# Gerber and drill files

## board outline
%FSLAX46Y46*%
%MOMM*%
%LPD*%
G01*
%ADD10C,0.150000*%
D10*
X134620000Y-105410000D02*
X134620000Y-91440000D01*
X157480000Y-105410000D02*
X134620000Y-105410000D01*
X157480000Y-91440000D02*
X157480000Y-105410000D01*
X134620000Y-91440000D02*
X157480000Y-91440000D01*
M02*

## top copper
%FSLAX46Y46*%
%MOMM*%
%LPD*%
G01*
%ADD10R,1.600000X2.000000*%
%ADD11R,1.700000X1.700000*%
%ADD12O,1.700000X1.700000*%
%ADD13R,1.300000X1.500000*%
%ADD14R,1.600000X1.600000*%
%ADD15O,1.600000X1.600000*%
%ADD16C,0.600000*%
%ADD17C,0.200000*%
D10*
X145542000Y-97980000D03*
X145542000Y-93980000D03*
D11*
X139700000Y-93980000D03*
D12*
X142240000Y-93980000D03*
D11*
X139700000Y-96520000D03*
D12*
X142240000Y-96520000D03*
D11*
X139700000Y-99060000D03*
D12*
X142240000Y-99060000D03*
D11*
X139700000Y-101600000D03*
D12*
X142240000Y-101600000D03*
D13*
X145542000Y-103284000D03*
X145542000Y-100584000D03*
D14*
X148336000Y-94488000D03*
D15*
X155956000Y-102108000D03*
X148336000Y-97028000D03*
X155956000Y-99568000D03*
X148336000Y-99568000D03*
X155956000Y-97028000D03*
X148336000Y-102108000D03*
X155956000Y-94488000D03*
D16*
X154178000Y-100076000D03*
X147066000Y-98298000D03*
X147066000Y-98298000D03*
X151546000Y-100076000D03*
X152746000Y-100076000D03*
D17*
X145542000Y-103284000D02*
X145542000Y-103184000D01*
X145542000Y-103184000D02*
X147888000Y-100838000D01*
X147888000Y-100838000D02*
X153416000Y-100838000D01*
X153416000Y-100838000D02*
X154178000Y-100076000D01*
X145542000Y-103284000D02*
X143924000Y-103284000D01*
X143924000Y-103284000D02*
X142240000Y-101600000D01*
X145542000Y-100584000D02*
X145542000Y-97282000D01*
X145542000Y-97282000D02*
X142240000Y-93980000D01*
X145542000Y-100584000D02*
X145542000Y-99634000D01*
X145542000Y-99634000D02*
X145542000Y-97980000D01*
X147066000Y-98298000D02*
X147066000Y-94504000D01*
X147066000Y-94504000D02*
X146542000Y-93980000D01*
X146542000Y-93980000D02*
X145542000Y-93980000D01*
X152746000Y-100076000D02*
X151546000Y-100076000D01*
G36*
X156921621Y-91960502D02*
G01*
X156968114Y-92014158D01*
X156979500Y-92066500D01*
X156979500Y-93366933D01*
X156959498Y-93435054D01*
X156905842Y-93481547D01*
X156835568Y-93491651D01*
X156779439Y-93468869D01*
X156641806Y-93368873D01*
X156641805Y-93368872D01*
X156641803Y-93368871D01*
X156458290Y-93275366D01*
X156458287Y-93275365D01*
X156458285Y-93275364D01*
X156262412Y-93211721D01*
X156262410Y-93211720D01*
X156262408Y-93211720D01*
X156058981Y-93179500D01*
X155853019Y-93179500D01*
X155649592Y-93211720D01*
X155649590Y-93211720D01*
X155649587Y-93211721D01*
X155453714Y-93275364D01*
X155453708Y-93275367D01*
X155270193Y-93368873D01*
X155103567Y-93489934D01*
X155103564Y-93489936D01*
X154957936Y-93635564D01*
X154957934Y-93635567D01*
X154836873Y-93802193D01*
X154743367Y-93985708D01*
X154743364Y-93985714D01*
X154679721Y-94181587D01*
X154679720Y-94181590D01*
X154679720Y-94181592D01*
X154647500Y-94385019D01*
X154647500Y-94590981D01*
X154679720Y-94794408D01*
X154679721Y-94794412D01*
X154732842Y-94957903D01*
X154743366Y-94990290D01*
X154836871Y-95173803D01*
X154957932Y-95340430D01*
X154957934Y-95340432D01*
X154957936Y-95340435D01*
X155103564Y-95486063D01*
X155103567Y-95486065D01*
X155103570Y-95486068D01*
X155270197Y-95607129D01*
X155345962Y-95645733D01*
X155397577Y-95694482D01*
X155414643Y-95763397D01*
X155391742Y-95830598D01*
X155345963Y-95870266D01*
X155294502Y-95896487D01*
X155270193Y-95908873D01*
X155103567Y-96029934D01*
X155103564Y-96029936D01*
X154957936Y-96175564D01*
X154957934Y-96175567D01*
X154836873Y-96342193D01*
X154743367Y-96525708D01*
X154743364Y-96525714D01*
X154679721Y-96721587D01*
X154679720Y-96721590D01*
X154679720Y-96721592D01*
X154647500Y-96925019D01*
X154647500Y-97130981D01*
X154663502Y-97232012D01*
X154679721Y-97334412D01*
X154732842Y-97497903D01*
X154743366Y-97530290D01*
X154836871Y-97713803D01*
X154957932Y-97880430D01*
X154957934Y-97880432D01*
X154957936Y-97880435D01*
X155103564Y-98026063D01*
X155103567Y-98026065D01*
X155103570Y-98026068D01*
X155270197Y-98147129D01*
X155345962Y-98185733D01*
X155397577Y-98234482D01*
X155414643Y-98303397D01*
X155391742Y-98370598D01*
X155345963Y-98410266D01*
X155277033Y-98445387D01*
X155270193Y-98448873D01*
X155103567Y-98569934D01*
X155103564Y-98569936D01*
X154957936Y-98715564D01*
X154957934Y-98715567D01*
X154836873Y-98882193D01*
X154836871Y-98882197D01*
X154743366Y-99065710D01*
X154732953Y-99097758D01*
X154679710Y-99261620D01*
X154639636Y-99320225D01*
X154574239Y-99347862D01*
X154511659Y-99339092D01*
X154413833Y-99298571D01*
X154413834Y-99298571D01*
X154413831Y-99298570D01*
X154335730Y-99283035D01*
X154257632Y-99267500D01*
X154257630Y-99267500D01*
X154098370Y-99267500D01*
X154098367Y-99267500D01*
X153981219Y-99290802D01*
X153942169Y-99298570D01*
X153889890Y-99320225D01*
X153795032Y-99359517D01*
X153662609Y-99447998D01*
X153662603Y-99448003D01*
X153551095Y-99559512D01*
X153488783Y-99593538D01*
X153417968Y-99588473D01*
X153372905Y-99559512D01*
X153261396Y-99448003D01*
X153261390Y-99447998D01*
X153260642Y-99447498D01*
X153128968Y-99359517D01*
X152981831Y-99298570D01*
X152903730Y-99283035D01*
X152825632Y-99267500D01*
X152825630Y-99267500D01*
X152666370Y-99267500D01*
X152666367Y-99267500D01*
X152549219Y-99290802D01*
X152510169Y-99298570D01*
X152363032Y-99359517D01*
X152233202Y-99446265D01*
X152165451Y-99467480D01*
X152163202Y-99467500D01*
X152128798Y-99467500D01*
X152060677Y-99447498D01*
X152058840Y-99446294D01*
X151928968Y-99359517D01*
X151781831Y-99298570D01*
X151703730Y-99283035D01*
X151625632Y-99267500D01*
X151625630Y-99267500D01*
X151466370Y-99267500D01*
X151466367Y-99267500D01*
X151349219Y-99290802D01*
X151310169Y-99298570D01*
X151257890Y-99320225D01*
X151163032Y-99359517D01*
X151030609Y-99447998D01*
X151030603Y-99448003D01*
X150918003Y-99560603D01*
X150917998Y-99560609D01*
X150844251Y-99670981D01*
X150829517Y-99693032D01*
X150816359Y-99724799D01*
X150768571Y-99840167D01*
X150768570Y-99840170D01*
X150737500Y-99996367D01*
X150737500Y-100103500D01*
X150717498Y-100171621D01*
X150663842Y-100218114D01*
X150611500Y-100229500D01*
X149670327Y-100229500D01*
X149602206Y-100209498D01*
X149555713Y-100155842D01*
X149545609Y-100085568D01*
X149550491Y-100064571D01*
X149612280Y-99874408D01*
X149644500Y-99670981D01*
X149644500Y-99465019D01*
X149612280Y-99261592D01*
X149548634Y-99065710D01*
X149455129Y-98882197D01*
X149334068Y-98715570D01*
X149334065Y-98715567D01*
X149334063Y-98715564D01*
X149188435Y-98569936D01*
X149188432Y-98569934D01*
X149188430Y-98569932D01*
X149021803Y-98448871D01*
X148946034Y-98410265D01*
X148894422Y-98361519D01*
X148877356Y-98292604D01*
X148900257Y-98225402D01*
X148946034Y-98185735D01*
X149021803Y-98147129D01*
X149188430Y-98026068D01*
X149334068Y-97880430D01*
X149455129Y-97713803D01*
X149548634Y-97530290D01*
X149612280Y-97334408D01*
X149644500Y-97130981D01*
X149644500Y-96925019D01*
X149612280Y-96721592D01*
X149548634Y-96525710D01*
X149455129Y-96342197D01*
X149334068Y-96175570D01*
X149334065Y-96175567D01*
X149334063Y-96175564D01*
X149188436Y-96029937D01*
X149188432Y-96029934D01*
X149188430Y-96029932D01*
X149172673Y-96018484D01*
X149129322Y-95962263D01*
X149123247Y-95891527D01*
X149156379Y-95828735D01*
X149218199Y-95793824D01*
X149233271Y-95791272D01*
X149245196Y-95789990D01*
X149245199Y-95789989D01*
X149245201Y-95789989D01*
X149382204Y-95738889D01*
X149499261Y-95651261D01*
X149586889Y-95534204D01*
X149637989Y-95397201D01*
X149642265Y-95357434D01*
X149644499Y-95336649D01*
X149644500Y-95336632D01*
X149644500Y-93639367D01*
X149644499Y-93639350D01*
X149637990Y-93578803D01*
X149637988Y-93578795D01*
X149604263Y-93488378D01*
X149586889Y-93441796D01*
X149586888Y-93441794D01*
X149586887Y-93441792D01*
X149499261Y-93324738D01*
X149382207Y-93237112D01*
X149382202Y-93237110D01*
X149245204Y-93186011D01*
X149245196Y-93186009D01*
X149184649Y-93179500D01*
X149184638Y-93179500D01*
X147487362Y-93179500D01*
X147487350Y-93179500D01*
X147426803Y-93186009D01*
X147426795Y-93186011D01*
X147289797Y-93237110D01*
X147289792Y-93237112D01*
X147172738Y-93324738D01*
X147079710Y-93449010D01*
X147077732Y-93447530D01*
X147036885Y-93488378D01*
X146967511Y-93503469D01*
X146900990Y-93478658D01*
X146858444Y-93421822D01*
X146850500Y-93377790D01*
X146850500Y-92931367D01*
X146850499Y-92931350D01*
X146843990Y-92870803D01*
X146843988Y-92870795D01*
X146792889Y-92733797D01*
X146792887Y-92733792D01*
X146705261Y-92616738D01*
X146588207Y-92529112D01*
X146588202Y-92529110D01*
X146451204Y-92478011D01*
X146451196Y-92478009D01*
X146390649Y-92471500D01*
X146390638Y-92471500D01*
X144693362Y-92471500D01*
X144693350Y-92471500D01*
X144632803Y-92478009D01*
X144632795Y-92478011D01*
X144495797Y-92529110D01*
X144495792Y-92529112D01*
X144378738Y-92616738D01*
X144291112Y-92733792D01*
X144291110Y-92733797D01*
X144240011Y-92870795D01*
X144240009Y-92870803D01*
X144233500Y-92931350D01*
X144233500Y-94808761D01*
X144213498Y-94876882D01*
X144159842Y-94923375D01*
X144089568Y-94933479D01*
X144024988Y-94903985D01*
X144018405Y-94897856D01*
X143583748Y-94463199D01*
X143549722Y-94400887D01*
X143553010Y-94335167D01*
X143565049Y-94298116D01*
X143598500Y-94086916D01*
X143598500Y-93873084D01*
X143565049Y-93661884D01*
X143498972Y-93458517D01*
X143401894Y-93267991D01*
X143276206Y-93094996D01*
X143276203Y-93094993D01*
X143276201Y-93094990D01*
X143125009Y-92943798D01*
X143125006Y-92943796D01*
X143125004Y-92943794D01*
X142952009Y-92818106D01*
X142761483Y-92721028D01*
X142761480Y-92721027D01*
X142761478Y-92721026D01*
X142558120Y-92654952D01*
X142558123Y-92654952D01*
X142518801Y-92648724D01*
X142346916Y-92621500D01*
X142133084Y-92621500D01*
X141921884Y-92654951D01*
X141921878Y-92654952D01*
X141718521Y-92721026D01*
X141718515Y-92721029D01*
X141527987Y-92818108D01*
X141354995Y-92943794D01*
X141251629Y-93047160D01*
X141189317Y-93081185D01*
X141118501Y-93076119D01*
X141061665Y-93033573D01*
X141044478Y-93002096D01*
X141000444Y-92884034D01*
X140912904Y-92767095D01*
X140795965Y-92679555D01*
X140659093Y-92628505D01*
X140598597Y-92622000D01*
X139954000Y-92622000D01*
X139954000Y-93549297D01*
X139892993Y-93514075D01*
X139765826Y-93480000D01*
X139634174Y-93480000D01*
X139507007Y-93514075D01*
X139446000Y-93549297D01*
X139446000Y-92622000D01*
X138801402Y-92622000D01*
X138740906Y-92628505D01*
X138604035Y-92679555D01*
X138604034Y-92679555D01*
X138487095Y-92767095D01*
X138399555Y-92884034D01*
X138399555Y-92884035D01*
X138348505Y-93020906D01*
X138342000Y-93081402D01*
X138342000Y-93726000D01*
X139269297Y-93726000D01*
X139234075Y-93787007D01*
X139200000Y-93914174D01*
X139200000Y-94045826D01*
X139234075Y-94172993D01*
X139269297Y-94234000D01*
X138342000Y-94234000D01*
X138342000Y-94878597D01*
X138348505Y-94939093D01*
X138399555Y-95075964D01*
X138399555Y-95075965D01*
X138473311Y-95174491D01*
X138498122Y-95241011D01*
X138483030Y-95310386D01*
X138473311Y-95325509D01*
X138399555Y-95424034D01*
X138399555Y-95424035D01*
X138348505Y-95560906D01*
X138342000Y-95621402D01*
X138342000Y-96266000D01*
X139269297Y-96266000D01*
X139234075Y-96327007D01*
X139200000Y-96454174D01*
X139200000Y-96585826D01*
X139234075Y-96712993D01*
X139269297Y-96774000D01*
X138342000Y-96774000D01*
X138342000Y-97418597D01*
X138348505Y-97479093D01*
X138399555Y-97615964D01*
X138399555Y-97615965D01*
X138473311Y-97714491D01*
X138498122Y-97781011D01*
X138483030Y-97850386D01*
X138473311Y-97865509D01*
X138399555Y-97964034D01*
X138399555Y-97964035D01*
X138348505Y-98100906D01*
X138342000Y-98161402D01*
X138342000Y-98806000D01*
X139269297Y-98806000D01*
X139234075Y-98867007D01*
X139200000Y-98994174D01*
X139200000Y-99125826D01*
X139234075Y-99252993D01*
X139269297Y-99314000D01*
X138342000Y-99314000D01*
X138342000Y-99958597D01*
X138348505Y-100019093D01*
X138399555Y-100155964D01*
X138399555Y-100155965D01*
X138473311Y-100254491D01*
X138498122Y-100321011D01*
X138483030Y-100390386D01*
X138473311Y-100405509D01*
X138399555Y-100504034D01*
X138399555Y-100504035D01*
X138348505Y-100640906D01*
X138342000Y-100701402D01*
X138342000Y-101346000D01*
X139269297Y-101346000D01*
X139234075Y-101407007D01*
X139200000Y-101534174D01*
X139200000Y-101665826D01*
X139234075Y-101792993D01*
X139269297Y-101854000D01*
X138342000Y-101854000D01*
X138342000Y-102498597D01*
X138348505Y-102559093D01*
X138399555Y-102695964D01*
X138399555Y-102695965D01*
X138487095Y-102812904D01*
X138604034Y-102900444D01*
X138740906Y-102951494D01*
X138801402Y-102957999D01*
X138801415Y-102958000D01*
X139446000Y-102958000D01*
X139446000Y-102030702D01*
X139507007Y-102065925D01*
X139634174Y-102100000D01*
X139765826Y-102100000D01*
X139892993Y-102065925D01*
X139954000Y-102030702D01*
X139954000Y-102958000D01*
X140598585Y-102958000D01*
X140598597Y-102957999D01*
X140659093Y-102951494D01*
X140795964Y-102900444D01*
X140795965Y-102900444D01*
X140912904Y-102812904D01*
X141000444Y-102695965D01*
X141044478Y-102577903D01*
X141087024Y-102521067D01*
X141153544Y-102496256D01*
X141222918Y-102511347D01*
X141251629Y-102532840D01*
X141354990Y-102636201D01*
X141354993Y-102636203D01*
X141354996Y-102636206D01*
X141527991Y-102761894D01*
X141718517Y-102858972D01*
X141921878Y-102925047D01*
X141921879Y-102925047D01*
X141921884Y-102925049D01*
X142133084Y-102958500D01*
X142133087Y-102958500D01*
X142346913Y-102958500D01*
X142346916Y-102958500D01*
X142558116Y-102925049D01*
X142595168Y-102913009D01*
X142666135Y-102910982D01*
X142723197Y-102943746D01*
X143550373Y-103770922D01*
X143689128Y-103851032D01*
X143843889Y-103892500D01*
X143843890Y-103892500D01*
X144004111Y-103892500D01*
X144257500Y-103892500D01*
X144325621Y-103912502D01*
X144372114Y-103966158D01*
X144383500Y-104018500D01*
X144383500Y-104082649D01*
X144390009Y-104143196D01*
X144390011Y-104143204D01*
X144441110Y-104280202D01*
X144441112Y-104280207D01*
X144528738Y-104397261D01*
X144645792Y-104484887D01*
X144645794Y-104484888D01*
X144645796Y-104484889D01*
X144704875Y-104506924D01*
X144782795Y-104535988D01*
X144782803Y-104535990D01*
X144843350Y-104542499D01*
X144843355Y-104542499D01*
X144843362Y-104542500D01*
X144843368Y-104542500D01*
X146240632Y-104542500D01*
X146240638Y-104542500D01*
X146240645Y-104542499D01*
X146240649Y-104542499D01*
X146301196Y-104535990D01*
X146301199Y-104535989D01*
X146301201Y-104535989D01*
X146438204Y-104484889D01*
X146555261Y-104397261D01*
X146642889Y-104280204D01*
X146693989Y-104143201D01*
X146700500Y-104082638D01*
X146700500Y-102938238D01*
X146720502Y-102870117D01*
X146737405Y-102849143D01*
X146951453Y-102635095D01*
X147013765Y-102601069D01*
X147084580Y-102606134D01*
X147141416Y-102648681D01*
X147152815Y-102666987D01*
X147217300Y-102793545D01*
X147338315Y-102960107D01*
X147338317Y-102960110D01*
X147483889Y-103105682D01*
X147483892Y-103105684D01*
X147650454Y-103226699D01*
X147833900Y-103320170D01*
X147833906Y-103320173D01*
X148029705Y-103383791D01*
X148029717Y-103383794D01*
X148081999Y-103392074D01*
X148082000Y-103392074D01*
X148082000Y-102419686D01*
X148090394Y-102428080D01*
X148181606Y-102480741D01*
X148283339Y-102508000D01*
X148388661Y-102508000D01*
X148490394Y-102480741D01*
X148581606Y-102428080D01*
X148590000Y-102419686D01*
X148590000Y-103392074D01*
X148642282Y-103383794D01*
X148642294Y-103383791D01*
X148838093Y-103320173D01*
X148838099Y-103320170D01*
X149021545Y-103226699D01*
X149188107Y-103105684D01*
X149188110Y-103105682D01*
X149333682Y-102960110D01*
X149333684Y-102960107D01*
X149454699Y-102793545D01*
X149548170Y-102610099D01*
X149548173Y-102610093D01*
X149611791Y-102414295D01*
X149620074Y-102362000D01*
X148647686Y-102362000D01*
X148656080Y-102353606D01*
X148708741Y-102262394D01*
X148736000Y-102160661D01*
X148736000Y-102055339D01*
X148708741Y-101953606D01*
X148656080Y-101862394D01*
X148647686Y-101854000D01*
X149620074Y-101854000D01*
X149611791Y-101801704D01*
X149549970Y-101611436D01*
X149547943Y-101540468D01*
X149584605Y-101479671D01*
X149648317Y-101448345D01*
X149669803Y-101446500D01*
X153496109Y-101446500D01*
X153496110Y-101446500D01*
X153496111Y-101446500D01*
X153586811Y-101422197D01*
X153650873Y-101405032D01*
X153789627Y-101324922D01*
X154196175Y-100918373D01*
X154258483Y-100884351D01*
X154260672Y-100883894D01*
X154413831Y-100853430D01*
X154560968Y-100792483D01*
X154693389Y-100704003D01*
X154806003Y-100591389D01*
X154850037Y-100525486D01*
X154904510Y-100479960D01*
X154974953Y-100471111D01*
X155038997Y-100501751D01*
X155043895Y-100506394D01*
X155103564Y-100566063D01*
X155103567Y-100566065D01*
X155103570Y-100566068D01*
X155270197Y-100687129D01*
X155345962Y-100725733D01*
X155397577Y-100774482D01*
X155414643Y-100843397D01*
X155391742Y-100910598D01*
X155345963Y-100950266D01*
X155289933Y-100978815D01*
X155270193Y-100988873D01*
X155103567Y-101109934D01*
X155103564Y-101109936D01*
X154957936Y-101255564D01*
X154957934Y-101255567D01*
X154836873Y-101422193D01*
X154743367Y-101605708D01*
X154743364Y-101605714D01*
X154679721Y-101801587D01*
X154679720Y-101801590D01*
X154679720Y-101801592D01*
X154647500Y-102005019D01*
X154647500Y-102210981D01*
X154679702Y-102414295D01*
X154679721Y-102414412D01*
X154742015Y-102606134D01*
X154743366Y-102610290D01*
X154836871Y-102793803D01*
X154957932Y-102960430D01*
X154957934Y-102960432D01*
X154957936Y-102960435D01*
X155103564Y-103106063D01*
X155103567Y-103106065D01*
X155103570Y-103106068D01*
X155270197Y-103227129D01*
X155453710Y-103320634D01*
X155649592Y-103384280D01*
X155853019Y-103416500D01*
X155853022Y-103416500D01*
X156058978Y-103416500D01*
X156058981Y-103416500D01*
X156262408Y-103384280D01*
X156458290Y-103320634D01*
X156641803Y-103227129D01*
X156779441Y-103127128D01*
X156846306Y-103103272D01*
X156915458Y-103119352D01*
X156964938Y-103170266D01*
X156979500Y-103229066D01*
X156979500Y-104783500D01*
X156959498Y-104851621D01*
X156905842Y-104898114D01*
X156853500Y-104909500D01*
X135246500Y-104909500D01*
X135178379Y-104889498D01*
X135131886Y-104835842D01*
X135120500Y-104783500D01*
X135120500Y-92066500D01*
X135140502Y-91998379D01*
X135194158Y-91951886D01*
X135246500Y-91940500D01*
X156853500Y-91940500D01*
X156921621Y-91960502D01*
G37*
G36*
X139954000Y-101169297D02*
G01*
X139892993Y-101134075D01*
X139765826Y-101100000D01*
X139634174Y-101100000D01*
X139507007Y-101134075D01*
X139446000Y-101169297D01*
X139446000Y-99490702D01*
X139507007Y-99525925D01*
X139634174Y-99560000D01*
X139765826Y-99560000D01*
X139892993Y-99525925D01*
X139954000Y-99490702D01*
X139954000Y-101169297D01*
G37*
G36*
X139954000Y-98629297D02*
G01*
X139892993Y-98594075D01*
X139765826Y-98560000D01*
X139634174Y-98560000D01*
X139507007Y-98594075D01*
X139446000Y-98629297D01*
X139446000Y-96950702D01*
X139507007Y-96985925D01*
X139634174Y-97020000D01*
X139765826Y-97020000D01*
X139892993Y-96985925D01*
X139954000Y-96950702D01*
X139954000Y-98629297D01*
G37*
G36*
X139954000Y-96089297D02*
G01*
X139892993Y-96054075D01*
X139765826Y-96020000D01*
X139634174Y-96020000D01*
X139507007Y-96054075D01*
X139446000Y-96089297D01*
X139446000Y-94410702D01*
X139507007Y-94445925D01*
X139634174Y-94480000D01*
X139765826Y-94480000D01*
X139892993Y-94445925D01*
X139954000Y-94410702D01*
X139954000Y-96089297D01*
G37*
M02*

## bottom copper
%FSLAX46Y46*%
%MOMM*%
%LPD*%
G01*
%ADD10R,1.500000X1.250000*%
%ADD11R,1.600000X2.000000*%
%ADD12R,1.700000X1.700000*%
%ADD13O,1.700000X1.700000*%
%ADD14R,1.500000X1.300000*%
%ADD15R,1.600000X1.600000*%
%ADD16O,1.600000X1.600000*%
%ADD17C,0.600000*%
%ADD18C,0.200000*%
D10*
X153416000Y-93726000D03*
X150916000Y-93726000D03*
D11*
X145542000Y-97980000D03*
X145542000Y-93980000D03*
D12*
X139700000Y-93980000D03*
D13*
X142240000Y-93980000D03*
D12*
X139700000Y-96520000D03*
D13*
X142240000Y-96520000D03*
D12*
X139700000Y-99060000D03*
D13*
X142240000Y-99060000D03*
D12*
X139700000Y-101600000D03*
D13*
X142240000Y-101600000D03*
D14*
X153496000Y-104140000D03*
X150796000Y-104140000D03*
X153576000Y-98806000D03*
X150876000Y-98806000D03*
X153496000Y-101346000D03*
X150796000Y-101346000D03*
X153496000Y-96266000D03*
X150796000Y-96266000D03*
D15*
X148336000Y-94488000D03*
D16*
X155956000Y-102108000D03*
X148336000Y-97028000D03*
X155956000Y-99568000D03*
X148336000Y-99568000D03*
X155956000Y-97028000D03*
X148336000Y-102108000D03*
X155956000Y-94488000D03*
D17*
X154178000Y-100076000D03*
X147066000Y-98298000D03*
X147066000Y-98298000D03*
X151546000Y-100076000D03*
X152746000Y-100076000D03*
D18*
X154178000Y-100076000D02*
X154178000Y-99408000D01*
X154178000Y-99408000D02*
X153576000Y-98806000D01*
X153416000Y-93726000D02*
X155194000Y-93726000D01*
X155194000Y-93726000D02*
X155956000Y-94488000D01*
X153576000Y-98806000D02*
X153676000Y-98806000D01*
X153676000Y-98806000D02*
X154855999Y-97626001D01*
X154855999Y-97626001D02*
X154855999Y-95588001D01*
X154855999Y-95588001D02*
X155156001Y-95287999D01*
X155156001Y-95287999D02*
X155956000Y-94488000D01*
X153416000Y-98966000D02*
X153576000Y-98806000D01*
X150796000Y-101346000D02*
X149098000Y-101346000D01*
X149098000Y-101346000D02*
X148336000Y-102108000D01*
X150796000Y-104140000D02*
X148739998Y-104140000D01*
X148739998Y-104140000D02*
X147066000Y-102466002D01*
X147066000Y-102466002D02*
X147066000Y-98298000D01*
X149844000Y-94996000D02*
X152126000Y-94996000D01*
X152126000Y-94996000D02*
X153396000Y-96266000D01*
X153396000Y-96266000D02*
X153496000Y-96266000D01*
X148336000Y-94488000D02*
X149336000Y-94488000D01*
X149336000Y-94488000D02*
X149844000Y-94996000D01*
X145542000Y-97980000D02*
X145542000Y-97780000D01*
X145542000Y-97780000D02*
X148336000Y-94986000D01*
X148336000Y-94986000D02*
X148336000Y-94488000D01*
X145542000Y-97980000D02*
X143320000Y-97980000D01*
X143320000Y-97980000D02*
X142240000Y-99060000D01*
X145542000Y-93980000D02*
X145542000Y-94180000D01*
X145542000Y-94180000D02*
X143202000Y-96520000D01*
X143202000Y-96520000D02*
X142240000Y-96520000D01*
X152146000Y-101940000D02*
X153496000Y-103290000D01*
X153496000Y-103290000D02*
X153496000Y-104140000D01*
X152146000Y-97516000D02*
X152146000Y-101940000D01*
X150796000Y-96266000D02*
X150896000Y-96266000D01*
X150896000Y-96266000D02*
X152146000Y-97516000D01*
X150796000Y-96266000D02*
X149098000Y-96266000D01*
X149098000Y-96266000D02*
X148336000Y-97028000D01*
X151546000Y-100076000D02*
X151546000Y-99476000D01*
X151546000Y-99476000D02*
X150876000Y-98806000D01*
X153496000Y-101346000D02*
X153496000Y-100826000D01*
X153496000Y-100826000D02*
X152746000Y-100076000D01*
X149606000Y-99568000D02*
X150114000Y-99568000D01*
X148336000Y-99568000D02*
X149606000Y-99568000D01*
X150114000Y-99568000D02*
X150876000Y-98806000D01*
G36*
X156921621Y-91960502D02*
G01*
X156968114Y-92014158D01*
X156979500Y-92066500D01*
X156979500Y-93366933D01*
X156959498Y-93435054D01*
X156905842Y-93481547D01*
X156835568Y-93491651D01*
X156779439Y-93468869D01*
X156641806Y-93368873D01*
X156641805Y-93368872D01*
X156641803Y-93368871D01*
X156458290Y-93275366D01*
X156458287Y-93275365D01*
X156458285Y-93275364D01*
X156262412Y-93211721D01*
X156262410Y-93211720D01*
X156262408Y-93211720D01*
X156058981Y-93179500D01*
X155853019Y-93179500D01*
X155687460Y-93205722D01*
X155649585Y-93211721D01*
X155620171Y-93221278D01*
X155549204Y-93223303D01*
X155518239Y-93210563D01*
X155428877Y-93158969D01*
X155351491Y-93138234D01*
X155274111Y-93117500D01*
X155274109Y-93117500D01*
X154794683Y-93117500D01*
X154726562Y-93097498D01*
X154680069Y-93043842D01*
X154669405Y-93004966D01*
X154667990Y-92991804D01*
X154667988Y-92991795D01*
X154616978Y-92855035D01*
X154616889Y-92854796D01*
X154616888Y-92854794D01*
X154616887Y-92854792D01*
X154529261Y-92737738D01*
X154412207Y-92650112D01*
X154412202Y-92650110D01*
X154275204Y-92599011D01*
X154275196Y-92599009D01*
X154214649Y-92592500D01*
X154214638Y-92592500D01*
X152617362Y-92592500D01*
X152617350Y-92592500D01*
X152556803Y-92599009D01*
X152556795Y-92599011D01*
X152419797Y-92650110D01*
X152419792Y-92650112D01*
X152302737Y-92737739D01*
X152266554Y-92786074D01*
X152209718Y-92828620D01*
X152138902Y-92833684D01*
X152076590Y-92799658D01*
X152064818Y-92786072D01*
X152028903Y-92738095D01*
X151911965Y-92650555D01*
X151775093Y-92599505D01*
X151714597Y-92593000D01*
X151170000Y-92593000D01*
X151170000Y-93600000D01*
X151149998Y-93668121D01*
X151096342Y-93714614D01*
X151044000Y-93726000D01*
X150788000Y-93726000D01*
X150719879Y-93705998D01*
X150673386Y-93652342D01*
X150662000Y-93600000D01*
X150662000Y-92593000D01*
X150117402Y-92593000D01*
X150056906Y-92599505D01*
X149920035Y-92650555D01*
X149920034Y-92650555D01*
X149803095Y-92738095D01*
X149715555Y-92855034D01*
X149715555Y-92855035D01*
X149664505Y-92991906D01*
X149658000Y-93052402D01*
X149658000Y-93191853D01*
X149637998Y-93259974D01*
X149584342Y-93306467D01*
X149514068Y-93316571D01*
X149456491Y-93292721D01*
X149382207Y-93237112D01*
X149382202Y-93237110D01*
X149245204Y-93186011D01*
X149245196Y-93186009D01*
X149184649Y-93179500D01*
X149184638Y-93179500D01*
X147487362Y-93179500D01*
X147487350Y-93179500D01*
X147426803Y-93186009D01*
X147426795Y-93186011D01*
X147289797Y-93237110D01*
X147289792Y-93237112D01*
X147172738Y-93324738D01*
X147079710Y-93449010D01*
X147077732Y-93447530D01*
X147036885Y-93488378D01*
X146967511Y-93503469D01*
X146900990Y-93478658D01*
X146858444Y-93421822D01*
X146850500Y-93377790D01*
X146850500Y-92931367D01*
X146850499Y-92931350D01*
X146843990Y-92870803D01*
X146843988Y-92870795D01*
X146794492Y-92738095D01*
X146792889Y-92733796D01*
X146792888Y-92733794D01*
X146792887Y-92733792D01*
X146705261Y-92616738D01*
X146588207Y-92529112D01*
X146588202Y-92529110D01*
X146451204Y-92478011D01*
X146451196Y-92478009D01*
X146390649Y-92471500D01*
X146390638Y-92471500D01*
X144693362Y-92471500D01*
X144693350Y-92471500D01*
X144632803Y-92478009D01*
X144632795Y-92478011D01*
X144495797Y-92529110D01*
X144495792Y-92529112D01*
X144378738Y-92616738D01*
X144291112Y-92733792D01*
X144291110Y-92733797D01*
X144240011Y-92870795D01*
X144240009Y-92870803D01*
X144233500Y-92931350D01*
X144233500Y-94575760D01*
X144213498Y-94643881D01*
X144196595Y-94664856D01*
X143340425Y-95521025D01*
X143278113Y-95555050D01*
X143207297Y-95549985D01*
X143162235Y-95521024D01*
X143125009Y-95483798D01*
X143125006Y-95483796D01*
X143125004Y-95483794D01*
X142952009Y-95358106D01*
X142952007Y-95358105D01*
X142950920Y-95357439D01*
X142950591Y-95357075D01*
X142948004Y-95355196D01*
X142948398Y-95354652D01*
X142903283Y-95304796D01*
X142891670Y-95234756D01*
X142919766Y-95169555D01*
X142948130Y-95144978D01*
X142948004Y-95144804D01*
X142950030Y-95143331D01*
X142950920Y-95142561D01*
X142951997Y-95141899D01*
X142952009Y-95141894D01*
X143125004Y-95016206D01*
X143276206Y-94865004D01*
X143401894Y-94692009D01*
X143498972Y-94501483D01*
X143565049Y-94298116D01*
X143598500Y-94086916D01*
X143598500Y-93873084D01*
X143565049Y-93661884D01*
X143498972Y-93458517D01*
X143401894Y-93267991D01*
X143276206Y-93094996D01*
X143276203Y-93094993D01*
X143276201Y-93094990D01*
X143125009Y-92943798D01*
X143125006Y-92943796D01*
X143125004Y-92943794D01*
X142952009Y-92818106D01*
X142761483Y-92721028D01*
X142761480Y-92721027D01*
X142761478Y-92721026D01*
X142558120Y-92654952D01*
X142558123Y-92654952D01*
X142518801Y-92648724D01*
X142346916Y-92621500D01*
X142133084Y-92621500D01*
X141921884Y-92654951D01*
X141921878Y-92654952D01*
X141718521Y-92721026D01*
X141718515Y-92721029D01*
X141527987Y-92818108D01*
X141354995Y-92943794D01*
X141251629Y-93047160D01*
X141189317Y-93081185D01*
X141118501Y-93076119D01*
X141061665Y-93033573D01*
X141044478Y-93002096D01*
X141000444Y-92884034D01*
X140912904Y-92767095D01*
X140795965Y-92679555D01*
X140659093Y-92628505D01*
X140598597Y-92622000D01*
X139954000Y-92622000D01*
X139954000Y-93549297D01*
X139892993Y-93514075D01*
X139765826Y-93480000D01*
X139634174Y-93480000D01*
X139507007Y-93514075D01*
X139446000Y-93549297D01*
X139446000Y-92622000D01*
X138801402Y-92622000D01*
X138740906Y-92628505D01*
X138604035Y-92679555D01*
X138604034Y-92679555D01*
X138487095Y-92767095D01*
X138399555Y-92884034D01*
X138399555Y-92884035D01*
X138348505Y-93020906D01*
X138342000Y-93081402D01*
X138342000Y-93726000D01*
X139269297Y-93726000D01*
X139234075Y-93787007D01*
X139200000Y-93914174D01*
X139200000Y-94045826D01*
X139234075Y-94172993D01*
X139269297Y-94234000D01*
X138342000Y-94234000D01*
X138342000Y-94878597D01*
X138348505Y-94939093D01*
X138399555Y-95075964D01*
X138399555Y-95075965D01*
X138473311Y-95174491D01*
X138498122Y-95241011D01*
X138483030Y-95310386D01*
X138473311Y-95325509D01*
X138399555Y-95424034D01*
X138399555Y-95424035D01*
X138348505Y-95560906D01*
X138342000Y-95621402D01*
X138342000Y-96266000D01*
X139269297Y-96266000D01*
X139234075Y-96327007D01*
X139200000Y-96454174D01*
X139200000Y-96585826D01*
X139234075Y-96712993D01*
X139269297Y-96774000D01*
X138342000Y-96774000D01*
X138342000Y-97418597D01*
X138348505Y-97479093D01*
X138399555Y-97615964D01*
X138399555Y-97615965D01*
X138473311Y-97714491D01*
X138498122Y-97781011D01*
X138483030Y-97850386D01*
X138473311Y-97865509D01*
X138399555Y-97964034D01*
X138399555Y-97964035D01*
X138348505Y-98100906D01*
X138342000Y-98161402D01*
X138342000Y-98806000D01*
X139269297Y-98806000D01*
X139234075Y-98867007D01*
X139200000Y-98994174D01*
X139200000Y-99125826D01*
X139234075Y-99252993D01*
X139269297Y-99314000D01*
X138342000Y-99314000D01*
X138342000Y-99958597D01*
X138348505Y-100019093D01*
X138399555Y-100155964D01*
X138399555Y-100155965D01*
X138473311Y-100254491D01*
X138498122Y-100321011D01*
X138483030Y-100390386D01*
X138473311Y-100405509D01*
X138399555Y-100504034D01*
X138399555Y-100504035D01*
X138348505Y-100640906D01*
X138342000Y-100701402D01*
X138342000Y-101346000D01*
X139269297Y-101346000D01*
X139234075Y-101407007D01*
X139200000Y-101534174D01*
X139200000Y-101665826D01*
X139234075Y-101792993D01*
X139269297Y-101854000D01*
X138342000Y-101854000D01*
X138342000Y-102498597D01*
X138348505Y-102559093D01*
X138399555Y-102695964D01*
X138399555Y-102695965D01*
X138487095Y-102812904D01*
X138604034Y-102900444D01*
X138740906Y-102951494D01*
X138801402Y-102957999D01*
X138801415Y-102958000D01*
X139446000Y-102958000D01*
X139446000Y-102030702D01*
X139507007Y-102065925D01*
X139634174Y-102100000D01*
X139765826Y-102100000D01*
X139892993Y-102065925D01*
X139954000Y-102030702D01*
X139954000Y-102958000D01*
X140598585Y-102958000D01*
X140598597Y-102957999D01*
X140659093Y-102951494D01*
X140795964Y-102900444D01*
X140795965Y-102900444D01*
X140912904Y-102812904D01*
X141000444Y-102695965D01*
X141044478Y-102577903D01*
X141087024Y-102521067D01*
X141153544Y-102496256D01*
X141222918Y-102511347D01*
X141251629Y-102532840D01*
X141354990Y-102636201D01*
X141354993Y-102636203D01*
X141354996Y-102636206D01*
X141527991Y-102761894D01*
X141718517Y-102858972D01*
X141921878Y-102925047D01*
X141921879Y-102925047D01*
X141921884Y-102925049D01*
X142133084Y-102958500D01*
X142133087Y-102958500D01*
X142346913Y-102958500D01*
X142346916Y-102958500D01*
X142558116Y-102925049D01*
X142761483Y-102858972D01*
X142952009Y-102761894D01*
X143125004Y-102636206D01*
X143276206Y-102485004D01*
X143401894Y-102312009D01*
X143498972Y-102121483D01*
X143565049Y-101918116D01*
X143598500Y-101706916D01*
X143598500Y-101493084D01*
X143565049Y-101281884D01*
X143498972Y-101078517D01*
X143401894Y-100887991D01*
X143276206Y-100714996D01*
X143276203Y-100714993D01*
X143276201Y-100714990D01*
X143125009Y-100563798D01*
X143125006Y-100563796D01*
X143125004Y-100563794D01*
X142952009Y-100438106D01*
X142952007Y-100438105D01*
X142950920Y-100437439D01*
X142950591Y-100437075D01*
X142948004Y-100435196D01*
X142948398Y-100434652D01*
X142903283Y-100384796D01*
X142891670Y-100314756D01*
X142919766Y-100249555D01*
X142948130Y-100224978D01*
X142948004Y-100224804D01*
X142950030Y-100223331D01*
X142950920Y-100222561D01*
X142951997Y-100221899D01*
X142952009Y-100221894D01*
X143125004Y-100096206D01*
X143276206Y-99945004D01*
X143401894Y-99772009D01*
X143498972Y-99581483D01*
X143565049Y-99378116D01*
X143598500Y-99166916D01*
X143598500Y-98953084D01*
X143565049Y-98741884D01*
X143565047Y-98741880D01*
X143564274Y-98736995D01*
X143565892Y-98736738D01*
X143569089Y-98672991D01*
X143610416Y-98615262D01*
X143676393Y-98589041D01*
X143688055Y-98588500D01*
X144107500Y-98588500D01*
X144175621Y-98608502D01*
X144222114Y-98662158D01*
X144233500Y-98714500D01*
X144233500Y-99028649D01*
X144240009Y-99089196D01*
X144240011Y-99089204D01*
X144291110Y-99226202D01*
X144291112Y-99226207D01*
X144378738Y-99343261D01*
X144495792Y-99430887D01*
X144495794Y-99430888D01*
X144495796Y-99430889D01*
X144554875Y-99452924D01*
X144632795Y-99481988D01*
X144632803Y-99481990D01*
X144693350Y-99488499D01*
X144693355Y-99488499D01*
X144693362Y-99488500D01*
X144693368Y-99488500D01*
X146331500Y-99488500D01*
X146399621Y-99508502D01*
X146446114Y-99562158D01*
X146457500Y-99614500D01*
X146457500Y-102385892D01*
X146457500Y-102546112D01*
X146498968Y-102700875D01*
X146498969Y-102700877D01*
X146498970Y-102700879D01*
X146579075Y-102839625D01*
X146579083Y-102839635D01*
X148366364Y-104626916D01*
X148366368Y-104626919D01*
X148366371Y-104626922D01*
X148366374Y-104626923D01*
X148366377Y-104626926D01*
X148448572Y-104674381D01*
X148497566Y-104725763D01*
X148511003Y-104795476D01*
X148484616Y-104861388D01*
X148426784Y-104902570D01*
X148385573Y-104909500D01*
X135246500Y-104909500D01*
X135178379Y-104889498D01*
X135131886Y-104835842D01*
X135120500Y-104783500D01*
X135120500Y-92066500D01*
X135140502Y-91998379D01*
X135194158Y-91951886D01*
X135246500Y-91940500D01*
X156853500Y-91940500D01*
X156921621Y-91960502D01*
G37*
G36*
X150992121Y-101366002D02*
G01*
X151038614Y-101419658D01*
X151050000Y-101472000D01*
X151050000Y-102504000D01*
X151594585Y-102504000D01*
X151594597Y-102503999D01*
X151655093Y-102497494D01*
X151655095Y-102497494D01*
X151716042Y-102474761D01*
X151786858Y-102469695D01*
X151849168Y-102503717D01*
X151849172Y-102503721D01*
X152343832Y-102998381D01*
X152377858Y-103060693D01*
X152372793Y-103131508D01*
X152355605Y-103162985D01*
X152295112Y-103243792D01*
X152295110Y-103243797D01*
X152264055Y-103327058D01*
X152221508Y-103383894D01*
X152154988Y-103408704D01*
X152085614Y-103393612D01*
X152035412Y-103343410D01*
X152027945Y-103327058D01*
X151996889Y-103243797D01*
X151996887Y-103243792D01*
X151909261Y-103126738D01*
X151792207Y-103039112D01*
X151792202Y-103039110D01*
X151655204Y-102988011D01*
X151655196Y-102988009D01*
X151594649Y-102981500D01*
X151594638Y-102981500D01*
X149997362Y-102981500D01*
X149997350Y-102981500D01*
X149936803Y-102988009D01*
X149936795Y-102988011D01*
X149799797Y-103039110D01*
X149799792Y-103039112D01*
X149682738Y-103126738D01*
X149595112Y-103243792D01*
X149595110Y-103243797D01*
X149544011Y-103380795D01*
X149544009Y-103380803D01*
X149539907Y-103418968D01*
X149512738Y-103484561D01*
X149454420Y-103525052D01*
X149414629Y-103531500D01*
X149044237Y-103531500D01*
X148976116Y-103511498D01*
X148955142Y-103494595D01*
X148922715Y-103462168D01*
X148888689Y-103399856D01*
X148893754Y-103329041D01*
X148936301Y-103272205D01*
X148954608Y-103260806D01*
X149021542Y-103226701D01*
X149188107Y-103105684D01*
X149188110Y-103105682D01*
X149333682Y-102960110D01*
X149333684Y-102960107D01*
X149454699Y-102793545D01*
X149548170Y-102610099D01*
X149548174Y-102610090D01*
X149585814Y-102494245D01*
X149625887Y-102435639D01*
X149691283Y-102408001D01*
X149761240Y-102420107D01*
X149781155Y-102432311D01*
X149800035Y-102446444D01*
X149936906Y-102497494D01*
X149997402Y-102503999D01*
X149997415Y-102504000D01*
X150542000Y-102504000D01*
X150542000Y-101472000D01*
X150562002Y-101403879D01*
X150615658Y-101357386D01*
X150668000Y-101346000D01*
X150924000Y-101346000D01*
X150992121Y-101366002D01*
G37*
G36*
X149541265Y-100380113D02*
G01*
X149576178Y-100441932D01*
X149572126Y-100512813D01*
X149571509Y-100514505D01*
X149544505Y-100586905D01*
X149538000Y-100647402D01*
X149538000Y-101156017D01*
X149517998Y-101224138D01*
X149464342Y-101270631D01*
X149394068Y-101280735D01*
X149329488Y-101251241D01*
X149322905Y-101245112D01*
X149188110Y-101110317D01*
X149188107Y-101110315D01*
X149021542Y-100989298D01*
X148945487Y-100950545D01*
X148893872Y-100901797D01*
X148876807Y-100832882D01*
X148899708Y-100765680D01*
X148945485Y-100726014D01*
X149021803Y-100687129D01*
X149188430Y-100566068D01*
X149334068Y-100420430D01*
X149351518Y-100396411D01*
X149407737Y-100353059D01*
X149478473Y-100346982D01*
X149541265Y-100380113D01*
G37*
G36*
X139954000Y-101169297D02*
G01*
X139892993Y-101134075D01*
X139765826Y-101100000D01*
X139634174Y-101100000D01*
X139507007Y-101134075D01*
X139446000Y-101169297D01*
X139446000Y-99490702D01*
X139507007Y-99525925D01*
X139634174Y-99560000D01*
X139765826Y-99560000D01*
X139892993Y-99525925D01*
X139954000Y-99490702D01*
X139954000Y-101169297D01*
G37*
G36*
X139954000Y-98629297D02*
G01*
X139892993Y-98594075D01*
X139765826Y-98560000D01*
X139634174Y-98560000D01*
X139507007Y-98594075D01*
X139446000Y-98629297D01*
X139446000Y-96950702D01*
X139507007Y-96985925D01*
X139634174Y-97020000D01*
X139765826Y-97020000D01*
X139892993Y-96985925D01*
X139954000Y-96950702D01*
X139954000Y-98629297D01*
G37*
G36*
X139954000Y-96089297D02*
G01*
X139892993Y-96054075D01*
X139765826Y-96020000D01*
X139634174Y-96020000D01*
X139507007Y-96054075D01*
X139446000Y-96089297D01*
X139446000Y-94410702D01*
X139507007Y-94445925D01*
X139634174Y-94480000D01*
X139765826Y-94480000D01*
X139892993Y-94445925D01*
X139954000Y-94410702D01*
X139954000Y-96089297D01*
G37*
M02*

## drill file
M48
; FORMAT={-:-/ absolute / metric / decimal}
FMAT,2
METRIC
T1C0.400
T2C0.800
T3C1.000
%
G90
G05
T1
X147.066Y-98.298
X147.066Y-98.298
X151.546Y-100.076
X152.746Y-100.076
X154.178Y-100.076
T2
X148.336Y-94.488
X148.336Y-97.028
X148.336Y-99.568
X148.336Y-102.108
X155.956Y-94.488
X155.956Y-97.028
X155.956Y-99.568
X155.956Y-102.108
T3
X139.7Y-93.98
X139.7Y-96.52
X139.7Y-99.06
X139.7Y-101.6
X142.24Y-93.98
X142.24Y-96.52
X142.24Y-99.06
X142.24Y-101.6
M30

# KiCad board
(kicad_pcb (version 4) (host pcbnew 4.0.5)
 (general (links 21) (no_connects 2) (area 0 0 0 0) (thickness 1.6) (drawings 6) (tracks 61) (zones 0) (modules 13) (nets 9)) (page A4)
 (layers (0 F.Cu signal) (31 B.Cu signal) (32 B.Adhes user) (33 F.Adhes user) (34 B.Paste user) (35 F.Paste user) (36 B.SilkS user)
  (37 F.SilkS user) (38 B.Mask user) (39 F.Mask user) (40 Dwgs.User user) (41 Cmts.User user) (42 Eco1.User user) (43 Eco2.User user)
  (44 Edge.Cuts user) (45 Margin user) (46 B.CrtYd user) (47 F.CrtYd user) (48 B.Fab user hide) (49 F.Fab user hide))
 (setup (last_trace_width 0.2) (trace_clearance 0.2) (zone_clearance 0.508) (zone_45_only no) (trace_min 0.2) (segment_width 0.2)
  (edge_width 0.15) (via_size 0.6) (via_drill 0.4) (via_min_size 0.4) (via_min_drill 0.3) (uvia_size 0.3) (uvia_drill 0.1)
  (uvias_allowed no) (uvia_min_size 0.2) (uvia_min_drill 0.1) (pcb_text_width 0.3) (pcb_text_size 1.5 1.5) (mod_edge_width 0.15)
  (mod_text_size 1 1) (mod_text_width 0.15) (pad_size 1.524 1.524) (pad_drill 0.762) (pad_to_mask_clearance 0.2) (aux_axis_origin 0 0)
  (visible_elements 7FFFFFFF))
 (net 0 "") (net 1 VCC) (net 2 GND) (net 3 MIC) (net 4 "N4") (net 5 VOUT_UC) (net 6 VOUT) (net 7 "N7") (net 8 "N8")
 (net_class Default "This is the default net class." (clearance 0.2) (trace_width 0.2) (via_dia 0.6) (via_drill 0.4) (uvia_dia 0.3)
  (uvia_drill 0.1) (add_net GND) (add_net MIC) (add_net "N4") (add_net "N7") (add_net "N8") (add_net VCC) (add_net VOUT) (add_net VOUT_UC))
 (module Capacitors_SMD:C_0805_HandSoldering (layer B.Cu) (at 152.166 93.726 180)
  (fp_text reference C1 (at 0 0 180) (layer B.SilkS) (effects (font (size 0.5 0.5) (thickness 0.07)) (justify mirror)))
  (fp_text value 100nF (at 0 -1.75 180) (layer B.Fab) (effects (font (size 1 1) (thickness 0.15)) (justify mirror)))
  (pad 1 smd rect (at -1.25 0 180) (size 1.5 1.25) (layers B.Cu B.Paste B.Mask) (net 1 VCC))
  (pad 2 smd rect (at 1.25 0 180) (size 1.5 1.25) (layers B.Cu B.Paste B.Mask) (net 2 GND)))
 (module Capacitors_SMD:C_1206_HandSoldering (layer F.Cu) (at 145.542 95.98 90)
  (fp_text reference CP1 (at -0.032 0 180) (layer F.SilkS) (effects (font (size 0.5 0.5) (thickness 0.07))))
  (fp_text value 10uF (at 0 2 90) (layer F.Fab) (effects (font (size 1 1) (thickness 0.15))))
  (pad 1 smd rect (at -2 0 90) (size 2 1.6) (layers F.Cu F.Paste F.Mask) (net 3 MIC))
  (pad 2 smd rect (at 2 0 90) (size 2 1.6) (layers F.Cu F.Paste F.Mask) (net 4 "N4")))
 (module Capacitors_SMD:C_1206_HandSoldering (layer B.Cu) (at 145.542 95.98 90)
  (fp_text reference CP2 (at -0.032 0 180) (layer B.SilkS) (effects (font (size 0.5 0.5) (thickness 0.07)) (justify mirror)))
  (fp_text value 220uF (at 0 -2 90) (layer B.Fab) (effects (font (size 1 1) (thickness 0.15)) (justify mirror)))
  (pad 1 smd rect (at -2 0 90) (size 2 1.6) (layers B.Cu B.Paste B.Mask) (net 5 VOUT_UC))
  (pad 2 smd rect (at 2 0 90) (size 2 1.6) (layers B.Cu B.Paste B.Mask) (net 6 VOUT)))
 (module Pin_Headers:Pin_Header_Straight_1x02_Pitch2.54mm (layer F.Cu) (at 139.7 93.98 90)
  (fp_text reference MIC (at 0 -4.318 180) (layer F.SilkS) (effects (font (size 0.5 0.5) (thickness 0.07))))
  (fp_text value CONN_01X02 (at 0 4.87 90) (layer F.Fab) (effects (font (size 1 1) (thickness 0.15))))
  (pad 1 thru_hole rect (at 0 0 90) (size 1.7 1.7) (drill 1) (layers *.Cu *.Mask) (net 2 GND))
  (pad 2 thru_hole oval (at 0 2.54 90) (size 1.7 1.7) (drill 1) (layers *.Cu *.Mask) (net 3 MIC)))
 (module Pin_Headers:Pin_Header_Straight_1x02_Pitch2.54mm (layer F.Cu) (at 139.7 96.52 90)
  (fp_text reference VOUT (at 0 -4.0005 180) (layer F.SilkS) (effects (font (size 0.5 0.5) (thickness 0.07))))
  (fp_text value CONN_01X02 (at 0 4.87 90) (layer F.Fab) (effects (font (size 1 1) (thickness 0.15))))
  (pad 1 thru_hole rect (at 0 0 90) (size 1.7 1.7) (drill 1) (layers *.Cu *.Mask) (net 2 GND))
  (pad 2 thru_hole oval (at 0 2.54 90) (size 1.7 1.7) (drill 1) (layers *.Cu *.Mask) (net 6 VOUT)))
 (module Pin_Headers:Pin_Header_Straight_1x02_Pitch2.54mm (layer F.Cu) (at 139.7 99.06 90)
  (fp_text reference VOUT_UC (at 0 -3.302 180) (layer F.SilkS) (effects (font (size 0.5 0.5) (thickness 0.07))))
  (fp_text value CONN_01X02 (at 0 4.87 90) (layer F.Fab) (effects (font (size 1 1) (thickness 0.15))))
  (pad 1 thru_hole rect (at 0 0 90) (size 1.7 1.7) (drill 1) (layers *.Cu *.Mask) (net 2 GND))
  (pad 2 thru_hole oval (at 0 2.54 90) (size 1.7 1.7) (drill 1) (layers *.Cu *.Mask) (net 5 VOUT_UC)))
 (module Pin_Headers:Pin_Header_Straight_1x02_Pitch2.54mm (layer F.Cu) (at 139.7 101.6 90)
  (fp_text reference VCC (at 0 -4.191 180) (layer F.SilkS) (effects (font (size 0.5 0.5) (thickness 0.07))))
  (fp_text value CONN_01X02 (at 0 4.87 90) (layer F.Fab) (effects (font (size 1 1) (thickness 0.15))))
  (pad 1 thru_hole rect (at 0 0 90) (size 1.7 1.7) (drill 1) (layers *.Cu *.Mask) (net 2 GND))
  (pad 2 thru_hole oval (at 0 2.54 90) (size 1.7 1.7) (drill 1) (layers *.Cu *.Mask) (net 1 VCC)))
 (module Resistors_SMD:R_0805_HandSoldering (layer F.Cu) (at 145.542 101.934 90)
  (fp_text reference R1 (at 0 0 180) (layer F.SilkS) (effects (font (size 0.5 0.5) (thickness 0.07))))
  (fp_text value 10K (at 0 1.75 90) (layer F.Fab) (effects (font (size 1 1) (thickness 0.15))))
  (pad 1 smd rect (at -1.35 0 90) (size 1.5 1.3) (layers F.Cu F.Paste F.Mask) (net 1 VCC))
  (pad 2 smd rect (at 1.35 0 90) (size 1.5 1.3) (layers F.Cu F.Paste F.Mask) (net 3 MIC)))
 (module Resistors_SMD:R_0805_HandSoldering (layer B.Cu) (at 152.146 104.14 180)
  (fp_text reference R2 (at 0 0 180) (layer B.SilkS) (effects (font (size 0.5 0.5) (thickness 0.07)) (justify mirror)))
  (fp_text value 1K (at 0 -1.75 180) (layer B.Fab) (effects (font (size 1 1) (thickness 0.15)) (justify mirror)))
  (pad 1 smd rect (at -1.35 0 180) (size 1.5 1.3) (layers B.Cu B.Paste B.Mask) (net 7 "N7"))
  (pad 2 smd rect (at 1.35 0 180) (size 1.5 1.3) (layers B.Cu B.Paste B.Mask) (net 4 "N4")))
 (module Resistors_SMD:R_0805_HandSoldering (layer B.Cu) (at 152.226 98.806 180)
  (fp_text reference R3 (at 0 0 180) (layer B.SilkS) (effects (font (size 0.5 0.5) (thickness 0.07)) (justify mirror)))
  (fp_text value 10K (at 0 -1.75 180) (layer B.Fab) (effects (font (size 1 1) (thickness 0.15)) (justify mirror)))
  (pad 1 smd rect (at -1.35 0 180) (size 1.5 1.3) (layers B.Cu B.Paste B.Mask) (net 1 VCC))
  (pad 2 smd rect (at 1.35 0 180) (size 1.5 1.3) (layers B.Cu B.Paste B.Mask) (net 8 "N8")))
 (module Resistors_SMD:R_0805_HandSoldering (layer B.Cu) (at 152.146 101.346 180)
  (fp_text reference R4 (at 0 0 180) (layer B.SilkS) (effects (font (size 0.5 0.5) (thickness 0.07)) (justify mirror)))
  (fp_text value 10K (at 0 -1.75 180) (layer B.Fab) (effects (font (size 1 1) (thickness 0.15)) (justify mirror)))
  (pad 1 smd rect (at -1.35 0 180) (size 1.5 1.3) (layers B.Cu B.Paste B.Mask) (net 8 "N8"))
  (pad 2 smd rect (at 1.35 0 180) (size 1.5 1.3) (layers B.Cu B.Paste B.Mask) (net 2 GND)))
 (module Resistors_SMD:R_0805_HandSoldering (layer B.Cu) (at 152.146 96.266 180)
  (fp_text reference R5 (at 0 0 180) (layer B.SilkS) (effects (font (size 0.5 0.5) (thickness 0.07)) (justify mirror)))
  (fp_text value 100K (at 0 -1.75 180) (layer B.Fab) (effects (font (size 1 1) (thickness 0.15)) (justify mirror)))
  (pad 1 smd rect (at -1.35 0 180) (size 1.5 1.3) (layers B.Cu B.Paste B.Mask) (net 5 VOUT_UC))
  (pad 2 smd rect (at 1.35 0 180) (size 1.5 1.3) (layers B.Cu B.Paste B.Mask) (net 7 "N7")))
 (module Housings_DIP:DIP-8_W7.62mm (layer F.Cu) (at 148.336 94.488)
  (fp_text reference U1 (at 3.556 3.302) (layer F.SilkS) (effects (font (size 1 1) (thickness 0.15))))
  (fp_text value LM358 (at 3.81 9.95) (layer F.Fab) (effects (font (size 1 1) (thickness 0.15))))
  (pad 1 thru_hole rect (at 0 0) (size 1.6 1.6) (drill 0.8) (layers *.Cu *.Mask) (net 5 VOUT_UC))
  (pad 5 thru_hole oval (at 7.62 7.62) (size 1.6 1.6) (drill 0.8) (layers *.Cu *.Mask))
  (pad 2 thru_hole oval (at 0 2.54) (size 1.6 1.6) (drill 0.8) (layers *.Cu *.Mask) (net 7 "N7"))
  (pad 6 thru_hole oval (at 7.62 5.08) (size 1.6 1.6) (drill 0.8) (layers *.Cu *.Mask))
  (pad 3 thru_hole oval (at 0 5.08) (size 1.6 1.6) (drill 0.8) (layers *.Cu *.Mask) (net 8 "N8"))
  (pad 7 thru_hole oval (at 7.62 2.54) (size 1.6 1.6) (drill 0.8) (layers *.Cu *.Mask))
  (pad 4 thru_hole oval (at 0 7.62) (size 1.6 1.6) (drill 0.8) (layers *.Cu *.Mask) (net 2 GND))
  (pad 8 thru_hole oval (at 7.62 0) (size 1.6 1.6) (drill 0.8) (layers *.Cu *.Mask) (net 1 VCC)))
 (gr_line (start 134.62 105.41) (end 134.62 91.44) (layer Edge.Cuts) (width 0.15))
 (gr_line (start 157.48 105.41) (end 134.62 105.41) (layer Edge.Cuts) (width 0.15))
 (gr_line (start 157.48 91.44) (end 157.48 105.41) (layer Edge.Cuts) (width 0.15))
 (gr_line (start 134.62 91.44) (end 157.48 91.44) (layer Edge.Cuts) (width 0.15))
 (segment (start 154.178 100.076) (end 154.178 99.408) (width 0.2) (layer B.Cu) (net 1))
 (segment (start 154.178 99.408) (end 153.576 98.806) (width 0.2) (layer B.Cu) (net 1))
 (segment (start 145.542 103.284) (end 145.542 103.184) (width 0.2) (layer F.Cu) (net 1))
 (segment (start 145.542 103.184) (end 147.888 100.838) (width 0.2) (layer F.Cu) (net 1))
 (segment (start 147.888 100.838) (end 153.416 100.838) (width 0.2) (layer F.Cu) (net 1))
 (segment (start 153.416 100.838) (end 154.178 100.076) (width 0.2) (layer F.Cu) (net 1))
 (segment (start 153.416 93.726) (end 155.194 93.726) (width 0.2) (layer B.Cu) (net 1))
 (segment (start 155.194 93.726) (end 155.956 94.488) (width 0.2) (layer B.Cu) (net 1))
 (segment (start 153.576 98.806) (end 153.676 98.806) (width 0.2) (layer B.Cu) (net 1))
 (segment (start 153.676 98.806) (end 154.855999 97.626001) (width 0.2) (layer B.Cu) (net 1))
 (segment (start 154.855999 97.626001) (end 154.855999 95.588001) (width 0.2) (layer B.Cu) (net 1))
 (segment (start 154.855999 95.588001) (end 155.156001 95.287999) (width 0.2) (layer B.Cu) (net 1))
 (segment (start 155.156001 95.287999) (end 155.956 94.488) (width 0.2) (layer B.Cu) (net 1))
 (segment (start 153.416 98.966) (end 153.576 98.806) (width 0.2) (layer B.Cu) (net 1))
 (via (at 154.178 100.076) (size 0.6) (drill 0.4) (layers F.Cu B.Cu) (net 1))
 (segment (start 145.542 103.284) (end 143.924 103.284) (width 0.2) (layer F.Cu) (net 1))
 (segment (start 143.924 103.284) (end 142.24 101.6) (width 0.2) (layer F.Cu) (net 1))
 (segment (start 150.796 101.346) (end 149.098 101.346) (width 0.2) (layer B.Cu) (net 2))
 (segment (start 149.098 101.346) (end 148.336 102.108) (width 0.2) (layer B.Cu) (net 2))
 (segment (start 145.542 100.584) (end 145.542 97.282) (width 0.2) (layer F.Cu) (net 3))
 (segment (start 145.542 97.282) (end 142.24 93.98) (width 0.2) (layer F.Cu) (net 3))
 (segment (start 145.542 100.584) (end 145.542 99.634) (width 0.2) (layer F.Cu) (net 3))
 (segment (start 145.542 99.634) (end 145.542 97.98) (width 0.2) (layer F.Cu) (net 3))
 (segment (start 147.066 98.298) (end 147.066 94.504) (width 0.2) (layer F.Cu) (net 4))
 (segment (start 147.066 94.504) (end 146.542 93.98) (width 0.2) (layer F.Cu) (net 4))
 (segment (start 146.542 93.98) (end 145.542 93.98) (width 0.2) (layer F.Cu) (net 4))
 (via (at 147.066 98.298) (size 0.6) (drill 0.4) (layers F.Cu B.Cu) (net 4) (status 1000000))
 (segment (start 150.796 104.14) (end 148.739998 104.14) (width 0.2) (layer B.Cu) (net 4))
 (segment (start 148.739998 104.14) (end 147.066 102.466002) (width 0.2) (layer B.Cu) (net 4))
 (segment (start 147.066 102.466002) (end 147.066 98.298) (width 0.2) (layer B.Cu) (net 4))
 (via (at 147.066 98.298) (size 0.6) (drill 0.4) (layers F.Cu B.Cu) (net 4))
 (segment (start 149.844 94.996) (end 152.126 94.996) (width 0.2) (layer B.Cu) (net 5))
 (segment (start 152.126 94.996) (end 153.396 96.266) (width 0.2) (layer B.Cu) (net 5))
 (segment (start 153.396 96.266) (end 153.496 96.266) (width 0.2) (layer B.Cu) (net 5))
 (segment (start 148.336 94.488) (end 149.336 94.488) (width 0.2) (layer B.Cu) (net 5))
 (segment (start 149.336 94.488) (end 149.844 94.996) (width 0.2) (layer B.Cu) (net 5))
 (segment (start 145.542 97.98) (end 145.542 97.78) (width 0.2) (layer B.Cu) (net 5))
 (segment (start 145.542 97.78) (end 148.336 94.986) (width 0.2) (layer B.Cu) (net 5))
 (segment (start 148.336 94.986) (end 148.336 94.488) (width 0.2) (layer B.Cu) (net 5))
 (segment (start 145.542 97.98) (end 143.32 97.98) (width 0.2) (layer B.Cu) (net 5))
 (segment (start 143.32 97.98) (end 142.24 99.06) (width 0.2) (layer B.Cu) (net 5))
 (segment (start 145.542 93.98) (end 145.542 94.18) (width 0.2) (layer B.Cu) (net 6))
 (segment (start 145.542 94.18) (end 143.202 96.52) (width 0.2) (layer B.Cu) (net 6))
 (segment (start 143.202 96.52) (end 142.24 96.52) (width 0.2) (layer B.Cu) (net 6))
 (segment (start 152.146 101.94) (end 153.496 103.29) (width 0.2) (layer B.Cu) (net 7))
 (segment (start 153.496 103.29) (end 153.496 104.14) (width 0.2) (layer B.Cu) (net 7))
 (segment (start 152.146 97.516) (end 152.146 101.94) (width 0.2) (layer B.Cu) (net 7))
 (segment (start 150.796 96.266) (end 150.896 96.266) (width 0.2) (layer B.Cu) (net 7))
 (segment (start 150.896 96.266) (end 152.146 97.516) (width 0.2) (layer B.Cu) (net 7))
 (segment (start 150.796 96.266) (end 149.098 96.266) (width 0.2) (layer B.Cu) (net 7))
 (segment (start 149.098 96.266) (end 148.336 97.028) (width 0.2) (layer B.Cu) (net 7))
 (segment (start 151.546 100.076) (end 151.546 99.476) (width 0.2) (layer B.Cu) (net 8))
 (segment (start 151.546 99.476) (end 150.876 98.806) (width 0.2) (layer B.Cu) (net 8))
 (segment (start 152.746 100.076) (end 151.546 100.076) (width 0.2) (layer F.Cu) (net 8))
 (via (at 151.546 100.076) (size 0.6) (drill 0.4) (layers F.Cu B.Cu) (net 8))
 (segment (start 153.496 101.346) (end 153.496 100.826) (width 0.2) (layer B.Cu) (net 8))
 (segment (start 153.496 100.826) (end 152.746 100.076) (width 0.2) (layer B.Cu) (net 8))
 (via (at 152.746 100.076) (size 0.6) (drill 0.4) (layers F.Cu B.Cu) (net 8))
 (segment (start 149.606 99.568) (end 150.114 99.568) (width 0.2) (layer B.Cu) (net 8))
 (segment (start 148.336 99.568) (end 149.606 99.568) (width 0.2) (layer B.Cu) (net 8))
 (segment (start 150.114 99.568) (end 150.876 98.806) (width 0.2) (layer B.Cu) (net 8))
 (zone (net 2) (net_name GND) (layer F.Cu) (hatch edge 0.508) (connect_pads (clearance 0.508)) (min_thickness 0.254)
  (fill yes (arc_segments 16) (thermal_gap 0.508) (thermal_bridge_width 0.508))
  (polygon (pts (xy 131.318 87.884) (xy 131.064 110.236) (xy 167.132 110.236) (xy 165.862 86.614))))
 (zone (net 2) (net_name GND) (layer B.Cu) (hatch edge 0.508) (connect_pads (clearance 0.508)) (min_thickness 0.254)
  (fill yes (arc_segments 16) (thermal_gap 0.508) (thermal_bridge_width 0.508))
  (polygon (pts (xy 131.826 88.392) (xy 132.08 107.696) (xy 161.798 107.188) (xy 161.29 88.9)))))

